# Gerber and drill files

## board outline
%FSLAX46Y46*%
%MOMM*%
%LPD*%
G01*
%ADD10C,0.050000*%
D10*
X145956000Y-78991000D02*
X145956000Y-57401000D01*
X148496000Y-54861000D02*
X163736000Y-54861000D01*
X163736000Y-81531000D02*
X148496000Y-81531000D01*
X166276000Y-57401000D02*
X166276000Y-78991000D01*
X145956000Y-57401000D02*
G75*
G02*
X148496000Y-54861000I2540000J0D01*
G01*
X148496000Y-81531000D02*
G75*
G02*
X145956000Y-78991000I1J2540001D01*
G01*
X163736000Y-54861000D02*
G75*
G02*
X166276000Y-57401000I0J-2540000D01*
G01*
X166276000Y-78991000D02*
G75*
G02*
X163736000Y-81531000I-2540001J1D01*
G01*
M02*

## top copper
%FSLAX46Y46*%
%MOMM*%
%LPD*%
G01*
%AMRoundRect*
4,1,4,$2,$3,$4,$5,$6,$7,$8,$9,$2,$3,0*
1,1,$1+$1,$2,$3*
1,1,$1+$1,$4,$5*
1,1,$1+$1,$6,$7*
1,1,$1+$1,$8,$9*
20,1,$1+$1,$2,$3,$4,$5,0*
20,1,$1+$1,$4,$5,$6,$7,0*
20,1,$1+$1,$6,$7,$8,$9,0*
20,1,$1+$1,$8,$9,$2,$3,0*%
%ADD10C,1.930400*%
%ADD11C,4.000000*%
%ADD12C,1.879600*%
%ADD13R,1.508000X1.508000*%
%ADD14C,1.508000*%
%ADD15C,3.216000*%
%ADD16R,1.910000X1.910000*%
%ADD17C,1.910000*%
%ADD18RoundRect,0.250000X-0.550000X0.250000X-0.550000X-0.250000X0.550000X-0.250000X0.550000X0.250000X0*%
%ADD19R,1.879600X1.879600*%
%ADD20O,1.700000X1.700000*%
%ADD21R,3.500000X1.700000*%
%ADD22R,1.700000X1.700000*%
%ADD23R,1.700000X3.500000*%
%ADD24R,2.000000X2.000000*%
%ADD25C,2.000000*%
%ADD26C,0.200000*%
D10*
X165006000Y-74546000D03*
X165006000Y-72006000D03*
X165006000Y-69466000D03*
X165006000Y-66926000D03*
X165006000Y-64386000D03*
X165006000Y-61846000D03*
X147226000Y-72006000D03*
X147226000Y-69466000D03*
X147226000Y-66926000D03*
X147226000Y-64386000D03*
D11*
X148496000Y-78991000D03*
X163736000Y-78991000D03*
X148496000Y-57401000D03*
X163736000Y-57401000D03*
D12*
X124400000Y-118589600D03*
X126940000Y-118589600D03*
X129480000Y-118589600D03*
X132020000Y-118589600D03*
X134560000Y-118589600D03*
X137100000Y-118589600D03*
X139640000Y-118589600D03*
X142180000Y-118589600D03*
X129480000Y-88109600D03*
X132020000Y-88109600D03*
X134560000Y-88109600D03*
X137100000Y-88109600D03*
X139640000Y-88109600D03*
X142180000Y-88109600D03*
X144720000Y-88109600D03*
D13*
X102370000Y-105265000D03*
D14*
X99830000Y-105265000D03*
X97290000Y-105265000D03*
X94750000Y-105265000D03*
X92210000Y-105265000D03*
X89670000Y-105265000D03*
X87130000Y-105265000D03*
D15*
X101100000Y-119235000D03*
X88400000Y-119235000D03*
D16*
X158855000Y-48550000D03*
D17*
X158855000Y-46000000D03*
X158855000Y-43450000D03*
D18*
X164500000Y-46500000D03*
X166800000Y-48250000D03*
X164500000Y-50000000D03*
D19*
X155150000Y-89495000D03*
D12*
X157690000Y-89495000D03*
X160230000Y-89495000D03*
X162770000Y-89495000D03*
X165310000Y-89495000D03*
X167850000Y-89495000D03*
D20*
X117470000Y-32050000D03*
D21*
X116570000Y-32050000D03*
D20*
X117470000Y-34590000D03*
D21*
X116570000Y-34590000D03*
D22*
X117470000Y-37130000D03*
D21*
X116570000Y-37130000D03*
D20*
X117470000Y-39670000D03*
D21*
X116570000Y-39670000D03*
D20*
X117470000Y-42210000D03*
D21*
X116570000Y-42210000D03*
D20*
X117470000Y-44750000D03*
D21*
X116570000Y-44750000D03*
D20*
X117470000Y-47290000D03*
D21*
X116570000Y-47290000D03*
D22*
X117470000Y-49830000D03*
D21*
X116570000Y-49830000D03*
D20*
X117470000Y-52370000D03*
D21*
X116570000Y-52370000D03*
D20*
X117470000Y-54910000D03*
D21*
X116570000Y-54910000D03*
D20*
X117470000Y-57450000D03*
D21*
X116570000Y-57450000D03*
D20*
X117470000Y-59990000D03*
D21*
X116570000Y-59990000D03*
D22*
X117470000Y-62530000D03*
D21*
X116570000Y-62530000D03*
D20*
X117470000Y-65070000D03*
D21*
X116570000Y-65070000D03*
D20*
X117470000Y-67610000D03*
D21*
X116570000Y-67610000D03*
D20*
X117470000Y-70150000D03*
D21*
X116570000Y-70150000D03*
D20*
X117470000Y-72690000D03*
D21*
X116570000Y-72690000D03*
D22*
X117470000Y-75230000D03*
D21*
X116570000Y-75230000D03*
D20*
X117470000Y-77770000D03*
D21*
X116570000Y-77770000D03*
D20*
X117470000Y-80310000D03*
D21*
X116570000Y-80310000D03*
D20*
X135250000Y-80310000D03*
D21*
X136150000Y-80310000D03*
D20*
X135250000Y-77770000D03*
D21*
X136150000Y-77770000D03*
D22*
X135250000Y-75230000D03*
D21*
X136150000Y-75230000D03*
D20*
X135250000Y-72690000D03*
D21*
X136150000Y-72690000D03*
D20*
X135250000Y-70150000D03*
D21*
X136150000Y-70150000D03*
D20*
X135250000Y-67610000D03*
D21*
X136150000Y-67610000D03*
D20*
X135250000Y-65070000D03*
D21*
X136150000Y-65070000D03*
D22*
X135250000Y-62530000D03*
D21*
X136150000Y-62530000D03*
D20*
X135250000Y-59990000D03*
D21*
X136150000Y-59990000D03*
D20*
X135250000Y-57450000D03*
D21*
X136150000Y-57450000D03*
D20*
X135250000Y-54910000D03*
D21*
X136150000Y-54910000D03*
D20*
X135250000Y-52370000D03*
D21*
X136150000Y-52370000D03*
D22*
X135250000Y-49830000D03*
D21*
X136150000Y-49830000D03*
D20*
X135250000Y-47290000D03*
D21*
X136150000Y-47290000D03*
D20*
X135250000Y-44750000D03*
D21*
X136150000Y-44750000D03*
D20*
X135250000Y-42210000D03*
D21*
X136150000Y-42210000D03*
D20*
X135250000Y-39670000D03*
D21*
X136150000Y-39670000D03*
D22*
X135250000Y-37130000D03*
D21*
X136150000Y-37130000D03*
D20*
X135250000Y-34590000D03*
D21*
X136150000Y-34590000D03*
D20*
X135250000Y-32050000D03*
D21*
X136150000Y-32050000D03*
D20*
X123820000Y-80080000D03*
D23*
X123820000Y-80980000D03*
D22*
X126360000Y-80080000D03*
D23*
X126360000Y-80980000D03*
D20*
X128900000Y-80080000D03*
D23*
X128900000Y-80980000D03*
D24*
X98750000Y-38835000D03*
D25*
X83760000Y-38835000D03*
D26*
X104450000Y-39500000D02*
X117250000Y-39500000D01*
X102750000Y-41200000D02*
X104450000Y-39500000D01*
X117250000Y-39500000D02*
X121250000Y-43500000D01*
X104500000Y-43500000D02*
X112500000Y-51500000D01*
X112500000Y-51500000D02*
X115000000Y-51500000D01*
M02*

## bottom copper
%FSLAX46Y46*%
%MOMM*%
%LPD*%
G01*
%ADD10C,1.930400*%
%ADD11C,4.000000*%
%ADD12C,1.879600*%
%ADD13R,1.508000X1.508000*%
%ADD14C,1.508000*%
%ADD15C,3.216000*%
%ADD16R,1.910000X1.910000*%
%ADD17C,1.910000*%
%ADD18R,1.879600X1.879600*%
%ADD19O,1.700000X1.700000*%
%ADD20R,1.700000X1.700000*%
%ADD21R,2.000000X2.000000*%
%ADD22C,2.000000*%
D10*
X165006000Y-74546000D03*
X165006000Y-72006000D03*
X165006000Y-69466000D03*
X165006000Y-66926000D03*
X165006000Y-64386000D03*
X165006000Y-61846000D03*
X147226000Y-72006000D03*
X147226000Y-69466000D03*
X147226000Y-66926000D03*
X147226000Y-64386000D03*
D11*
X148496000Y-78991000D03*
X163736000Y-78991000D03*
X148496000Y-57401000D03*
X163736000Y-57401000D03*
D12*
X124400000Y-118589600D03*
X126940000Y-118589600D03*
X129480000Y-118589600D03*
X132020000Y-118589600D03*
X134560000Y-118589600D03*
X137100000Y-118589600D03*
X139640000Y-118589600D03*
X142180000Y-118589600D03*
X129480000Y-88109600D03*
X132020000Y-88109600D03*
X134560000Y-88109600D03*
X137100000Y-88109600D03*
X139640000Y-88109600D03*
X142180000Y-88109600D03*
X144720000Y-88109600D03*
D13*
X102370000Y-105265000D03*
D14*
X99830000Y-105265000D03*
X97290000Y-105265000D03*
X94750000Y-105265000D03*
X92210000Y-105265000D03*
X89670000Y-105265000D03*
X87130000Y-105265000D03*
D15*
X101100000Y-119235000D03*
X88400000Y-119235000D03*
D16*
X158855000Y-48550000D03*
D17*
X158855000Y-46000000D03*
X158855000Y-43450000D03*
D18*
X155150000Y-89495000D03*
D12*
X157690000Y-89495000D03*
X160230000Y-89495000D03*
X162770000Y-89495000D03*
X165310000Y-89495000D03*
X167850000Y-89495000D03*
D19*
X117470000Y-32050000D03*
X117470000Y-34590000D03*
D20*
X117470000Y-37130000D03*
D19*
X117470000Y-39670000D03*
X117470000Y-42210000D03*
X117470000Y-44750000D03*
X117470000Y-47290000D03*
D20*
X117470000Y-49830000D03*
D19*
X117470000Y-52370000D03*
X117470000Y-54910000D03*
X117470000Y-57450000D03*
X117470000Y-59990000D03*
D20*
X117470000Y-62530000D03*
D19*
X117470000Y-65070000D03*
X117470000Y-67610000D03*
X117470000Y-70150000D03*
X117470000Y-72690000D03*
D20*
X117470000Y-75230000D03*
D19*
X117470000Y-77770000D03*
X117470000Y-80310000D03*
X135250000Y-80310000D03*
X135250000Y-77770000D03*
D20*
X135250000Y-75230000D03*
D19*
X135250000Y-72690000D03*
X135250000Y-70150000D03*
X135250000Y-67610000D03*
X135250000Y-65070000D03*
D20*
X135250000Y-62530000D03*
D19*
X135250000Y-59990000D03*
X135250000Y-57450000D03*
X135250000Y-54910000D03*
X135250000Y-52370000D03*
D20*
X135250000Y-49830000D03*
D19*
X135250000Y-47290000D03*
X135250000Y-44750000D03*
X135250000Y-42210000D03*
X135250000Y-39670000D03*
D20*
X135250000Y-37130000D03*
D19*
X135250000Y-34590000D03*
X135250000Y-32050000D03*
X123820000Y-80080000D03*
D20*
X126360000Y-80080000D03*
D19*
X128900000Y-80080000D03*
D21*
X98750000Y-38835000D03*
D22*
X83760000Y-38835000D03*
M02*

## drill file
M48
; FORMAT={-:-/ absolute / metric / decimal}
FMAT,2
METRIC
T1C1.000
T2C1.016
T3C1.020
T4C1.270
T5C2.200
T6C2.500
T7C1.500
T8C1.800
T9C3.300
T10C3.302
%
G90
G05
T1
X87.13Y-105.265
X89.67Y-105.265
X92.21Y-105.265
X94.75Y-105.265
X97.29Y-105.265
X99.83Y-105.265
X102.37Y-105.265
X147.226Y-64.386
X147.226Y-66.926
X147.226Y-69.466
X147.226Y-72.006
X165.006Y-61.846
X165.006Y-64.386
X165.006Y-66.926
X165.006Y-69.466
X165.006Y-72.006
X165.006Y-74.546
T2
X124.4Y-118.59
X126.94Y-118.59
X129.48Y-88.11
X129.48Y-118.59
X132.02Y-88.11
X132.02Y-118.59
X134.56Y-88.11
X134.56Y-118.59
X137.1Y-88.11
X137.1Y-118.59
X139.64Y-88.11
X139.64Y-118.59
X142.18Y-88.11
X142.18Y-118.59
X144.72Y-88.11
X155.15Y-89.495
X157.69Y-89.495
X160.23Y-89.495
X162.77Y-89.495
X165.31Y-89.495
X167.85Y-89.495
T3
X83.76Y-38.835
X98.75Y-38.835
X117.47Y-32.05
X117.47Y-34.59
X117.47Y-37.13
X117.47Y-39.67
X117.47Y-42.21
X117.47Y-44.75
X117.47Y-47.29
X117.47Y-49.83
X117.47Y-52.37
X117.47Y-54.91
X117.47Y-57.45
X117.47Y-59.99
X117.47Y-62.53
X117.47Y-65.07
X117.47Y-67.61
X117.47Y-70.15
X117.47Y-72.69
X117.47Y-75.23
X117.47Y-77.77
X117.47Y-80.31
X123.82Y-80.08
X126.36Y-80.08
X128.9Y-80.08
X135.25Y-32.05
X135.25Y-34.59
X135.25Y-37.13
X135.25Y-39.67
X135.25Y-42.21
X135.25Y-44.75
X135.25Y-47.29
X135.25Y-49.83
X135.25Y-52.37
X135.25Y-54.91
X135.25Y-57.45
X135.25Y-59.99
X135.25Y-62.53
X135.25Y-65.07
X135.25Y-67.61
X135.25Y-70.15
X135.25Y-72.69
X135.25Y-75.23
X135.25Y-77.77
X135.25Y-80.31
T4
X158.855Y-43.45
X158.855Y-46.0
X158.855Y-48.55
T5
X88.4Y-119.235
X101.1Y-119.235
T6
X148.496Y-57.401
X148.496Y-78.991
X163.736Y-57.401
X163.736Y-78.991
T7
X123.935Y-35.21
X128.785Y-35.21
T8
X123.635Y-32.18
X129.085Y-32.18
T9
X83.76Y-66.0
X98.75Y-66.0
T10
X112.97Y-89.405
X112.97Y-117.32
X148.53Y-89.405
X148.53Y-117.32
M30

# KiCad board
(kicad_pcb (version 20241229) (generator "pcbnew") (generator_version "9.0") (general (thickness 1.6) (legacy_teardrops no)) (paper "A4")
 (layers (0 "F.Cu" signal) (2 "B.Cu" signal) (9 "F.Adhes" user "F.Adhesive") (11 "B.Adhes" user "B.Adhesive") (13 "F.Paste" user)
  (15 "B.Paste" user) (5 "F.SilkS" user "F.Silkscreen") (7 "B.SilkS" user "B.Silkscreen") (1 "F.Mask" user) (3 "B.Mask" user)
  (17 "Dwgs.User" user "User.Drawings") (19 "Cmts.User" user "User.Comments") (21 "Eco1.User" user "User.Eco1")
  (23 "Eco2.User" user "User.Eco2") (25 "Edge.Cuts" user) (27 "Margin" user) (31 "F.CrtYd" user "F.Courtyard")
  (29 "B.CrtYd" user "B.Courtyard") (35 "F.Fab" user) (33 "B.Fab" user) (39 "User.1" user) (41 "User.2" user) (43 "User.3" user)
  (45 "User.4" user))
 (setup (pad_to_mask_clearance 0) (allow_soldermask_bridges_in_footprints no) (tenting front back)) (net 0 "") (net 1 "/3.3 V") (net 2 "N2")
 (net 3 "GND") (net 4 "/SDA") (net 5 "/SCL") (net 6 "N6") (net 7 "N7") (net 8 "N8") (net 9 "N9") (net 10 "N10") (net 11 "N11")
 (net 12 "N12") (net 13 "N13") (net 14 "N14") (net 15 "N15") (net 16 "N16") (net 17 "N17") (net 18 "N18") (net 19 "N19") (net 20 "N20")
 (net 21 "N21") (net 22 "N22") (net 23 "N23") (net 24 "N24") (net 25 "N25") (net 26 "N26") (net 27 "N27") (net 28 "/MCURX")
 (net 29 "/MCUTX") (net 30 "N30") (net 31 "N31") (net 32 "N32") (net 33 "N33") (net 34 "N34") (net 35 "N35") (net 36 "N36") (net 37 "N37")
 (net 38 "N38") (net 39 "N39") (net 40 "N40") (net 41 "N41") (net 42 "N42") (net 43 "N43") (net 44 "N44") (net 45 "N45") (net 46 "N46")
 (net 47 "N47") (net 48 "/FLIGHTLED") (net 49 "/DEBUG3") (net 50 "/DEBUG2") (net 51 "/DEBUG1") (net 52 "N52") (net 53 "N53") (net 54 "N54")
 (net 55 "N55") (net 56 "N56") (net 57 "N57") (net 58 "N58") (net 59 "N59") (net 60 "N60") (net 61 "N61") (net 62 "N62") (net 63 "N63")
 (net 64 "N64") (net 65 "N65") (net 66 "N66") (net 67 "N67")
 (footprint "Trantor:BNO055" (layer "F.Cu") (at 156.75 67.75 90)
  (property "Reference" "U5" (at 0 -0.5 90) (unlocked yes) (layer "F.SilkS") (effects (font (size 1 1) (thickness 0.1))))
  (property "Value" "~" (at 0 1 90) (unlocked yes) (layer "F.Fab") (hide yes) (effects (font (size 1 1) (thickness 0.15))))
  (fp_line (start -11.241 -10.794) (end 10.349 -10.794) (stroke (width 0.05) (type solid)) (layer "Edge.Cuts"))
  (fp_line (start 12.889 -8.254) (end 12.889 6.986) (stroke (width 0.05) (type solid)) (layer "Edge.Cuts"))
  (fp_line (start -13.781 6.986) (end -13.781 -8.254) (stroke (width 0.05) (type solid)) (layer "Edge.Cuts"))
  (fp_line (start 10.349 9.526) (end -11.241 9.526) (stroke (width 0.05) (type solid)) (layer "Edge.Cuts"))
  (fp_arc (start 10.349 -10.794) (mid 12.145051 -10.050051) (end 12.889 -8.254) (stroke (width 0.05) (type solid)) (layer "Edge.Cuts"))
  (fp_arc (start -13.781 -8.254) (mid -13.037051 -10.050051) (end -11.241 -10.794) (stroke (width 0.05) (type solid)) (layer "Edge.Cuts"))
  (fp_arc (start 12.889 6.986) (mid 12.145051 8.782051) (end 10.349 9.526) (stroke (width 0.05) (type solid)) (layer "Edge.Cuts"))
  (fp_arc (start -11.241 9.526) (mid -13.037051 8.782051) (end -13.781 6.986) (stroke (width 0.05) (type solid)) (layer "Edge.Cuts"))
  (pad "1" thru_hole circle (at -6.796 8.256 180) (size 1.9304 1.9304) (drill 1) (layers "*.Cu" "*.Mask") (remove_unused_layers no)
   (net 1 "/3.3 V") (solder_mask_margin 0.0508) (thermal_bridge_angle 0))
  (pad "2" thru_hole circle (at -4.256 8.256 180) (size 1.9304 1.9304) (drill 1) (layers "*.Cu" "*.Mask") (remove_unused_layers no)
   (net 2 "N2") (solder_mask_margin 0.0508) (thermal_bridge_angle 0))
  (pad "3" thru_hole circle (at -1.716 8.256 180) (size 1.9304 1.9304) (drill 1) (layers "*.Cu" "*.Mask") (remove_unused_layers no)
   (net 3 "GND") (solder_mask_margin 0.0508) (thermal_bridge_angle 0))
  (pad "4" thru_hole circle (at 0.824 8.256 180) (size 1.9304 1.9304) (drill 1) (layers "*.Cu" "*.Mask") (remove_unused_layers no)
   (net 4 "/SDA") (solder_mask_margin 0.0508) (thermal_bridge_angle 0))
  (pad "5" thru_hole circle (at 3.364 8.256 180) (size 1.9304 1.9304) (drill 1) (layers "*.Cu" "*.Mask") (remove_unused_layers no)
   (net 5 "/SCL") (solder_mask_margin 0.0508) (thermal_bridge_angle 0))
  (pad "6" thru_hole circle (at 5.904 8.256 180) (size 1.9304 1.9304) (drill 1) (layers "*.Cu" "*.Mask") (remove_unused_layers no)
   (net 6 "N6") (solder_mask_margin 0.0508) (thermal_bridge_angle 0))
  (pad "7" thru_hole circle (at -4.256 -9.524 180) (size 1.9304 1.9304) (drill 1) (layers "*.Cu" "*.Mask") (remove_unused_layers no)
   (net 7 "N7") (solder_mask_margin 0.0508) (thermal_bridge_angle 0))
  (pad "8" thru_hole circle (at -1.716 -9.524 180) (size 1.9304 1.9304) (drill 1) (layers "*.Cu" "*.Mask") (remove_unused_layers no)
   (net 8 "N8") (solder_mask_margin 0.0508) (thermal_bridge_angle 0))
  (pad "9" thru_hole circle (at 0.824 -9.524 180) (size 1.9304 1.9304) (drill 1) (layers "*.Cu" "*.Mask") (remove_unused_layers no)
   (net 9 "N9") (solder_mask_margin 0.0508) (thermal_bridge_angle 0))
  (pad "10" thru_hole circle (at 3.364 -9.524 180) (size 1.9304 1.9304) (drill 1) (layers "*.Cu" "*.Mask") (remove_unused_layers no)
   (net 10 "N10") (solder_mask_margin 0.0508) (thermal_bridge_angle 0))
  (pad "P$1" thru_hole circle (at -11.241 -8.254 90) (size 4 4) (drill 2.5) (layers "*.Cu" "*.Mask") (remove_unused_layers no)
   (solder_mask_margin 0.0508) (thermal_bridge_angle 0))
  (pad "P$1" thru_hole circle (at -11.241 6.986 90) (size 4 4) (drill 2.5) (layers "*.Cu" "*.Mask") (remove_unused_layers no)
   (solder_mask_margin 0.0508) (thermal_bridge_angle 0))
  (pad "P$1" thru_hole circle (at 10.349 -8.254 90) (size 4 4) (drill 2.5) (layers "*.Cu" "*.Mask") (remove_unused_layers no)
   (solder_mask_margin 0.0508) (thermal_bridge_angle 0))
  (pad "P$1" thru_hole circle (at 10.349 6.986 90) (size 4 4) (drill 2.5) (layers "*.Cu" "*.Mask") (remove_unused_layers no)
   (solder_mask_margin 0.0508) (thermal_bridge_angle 0))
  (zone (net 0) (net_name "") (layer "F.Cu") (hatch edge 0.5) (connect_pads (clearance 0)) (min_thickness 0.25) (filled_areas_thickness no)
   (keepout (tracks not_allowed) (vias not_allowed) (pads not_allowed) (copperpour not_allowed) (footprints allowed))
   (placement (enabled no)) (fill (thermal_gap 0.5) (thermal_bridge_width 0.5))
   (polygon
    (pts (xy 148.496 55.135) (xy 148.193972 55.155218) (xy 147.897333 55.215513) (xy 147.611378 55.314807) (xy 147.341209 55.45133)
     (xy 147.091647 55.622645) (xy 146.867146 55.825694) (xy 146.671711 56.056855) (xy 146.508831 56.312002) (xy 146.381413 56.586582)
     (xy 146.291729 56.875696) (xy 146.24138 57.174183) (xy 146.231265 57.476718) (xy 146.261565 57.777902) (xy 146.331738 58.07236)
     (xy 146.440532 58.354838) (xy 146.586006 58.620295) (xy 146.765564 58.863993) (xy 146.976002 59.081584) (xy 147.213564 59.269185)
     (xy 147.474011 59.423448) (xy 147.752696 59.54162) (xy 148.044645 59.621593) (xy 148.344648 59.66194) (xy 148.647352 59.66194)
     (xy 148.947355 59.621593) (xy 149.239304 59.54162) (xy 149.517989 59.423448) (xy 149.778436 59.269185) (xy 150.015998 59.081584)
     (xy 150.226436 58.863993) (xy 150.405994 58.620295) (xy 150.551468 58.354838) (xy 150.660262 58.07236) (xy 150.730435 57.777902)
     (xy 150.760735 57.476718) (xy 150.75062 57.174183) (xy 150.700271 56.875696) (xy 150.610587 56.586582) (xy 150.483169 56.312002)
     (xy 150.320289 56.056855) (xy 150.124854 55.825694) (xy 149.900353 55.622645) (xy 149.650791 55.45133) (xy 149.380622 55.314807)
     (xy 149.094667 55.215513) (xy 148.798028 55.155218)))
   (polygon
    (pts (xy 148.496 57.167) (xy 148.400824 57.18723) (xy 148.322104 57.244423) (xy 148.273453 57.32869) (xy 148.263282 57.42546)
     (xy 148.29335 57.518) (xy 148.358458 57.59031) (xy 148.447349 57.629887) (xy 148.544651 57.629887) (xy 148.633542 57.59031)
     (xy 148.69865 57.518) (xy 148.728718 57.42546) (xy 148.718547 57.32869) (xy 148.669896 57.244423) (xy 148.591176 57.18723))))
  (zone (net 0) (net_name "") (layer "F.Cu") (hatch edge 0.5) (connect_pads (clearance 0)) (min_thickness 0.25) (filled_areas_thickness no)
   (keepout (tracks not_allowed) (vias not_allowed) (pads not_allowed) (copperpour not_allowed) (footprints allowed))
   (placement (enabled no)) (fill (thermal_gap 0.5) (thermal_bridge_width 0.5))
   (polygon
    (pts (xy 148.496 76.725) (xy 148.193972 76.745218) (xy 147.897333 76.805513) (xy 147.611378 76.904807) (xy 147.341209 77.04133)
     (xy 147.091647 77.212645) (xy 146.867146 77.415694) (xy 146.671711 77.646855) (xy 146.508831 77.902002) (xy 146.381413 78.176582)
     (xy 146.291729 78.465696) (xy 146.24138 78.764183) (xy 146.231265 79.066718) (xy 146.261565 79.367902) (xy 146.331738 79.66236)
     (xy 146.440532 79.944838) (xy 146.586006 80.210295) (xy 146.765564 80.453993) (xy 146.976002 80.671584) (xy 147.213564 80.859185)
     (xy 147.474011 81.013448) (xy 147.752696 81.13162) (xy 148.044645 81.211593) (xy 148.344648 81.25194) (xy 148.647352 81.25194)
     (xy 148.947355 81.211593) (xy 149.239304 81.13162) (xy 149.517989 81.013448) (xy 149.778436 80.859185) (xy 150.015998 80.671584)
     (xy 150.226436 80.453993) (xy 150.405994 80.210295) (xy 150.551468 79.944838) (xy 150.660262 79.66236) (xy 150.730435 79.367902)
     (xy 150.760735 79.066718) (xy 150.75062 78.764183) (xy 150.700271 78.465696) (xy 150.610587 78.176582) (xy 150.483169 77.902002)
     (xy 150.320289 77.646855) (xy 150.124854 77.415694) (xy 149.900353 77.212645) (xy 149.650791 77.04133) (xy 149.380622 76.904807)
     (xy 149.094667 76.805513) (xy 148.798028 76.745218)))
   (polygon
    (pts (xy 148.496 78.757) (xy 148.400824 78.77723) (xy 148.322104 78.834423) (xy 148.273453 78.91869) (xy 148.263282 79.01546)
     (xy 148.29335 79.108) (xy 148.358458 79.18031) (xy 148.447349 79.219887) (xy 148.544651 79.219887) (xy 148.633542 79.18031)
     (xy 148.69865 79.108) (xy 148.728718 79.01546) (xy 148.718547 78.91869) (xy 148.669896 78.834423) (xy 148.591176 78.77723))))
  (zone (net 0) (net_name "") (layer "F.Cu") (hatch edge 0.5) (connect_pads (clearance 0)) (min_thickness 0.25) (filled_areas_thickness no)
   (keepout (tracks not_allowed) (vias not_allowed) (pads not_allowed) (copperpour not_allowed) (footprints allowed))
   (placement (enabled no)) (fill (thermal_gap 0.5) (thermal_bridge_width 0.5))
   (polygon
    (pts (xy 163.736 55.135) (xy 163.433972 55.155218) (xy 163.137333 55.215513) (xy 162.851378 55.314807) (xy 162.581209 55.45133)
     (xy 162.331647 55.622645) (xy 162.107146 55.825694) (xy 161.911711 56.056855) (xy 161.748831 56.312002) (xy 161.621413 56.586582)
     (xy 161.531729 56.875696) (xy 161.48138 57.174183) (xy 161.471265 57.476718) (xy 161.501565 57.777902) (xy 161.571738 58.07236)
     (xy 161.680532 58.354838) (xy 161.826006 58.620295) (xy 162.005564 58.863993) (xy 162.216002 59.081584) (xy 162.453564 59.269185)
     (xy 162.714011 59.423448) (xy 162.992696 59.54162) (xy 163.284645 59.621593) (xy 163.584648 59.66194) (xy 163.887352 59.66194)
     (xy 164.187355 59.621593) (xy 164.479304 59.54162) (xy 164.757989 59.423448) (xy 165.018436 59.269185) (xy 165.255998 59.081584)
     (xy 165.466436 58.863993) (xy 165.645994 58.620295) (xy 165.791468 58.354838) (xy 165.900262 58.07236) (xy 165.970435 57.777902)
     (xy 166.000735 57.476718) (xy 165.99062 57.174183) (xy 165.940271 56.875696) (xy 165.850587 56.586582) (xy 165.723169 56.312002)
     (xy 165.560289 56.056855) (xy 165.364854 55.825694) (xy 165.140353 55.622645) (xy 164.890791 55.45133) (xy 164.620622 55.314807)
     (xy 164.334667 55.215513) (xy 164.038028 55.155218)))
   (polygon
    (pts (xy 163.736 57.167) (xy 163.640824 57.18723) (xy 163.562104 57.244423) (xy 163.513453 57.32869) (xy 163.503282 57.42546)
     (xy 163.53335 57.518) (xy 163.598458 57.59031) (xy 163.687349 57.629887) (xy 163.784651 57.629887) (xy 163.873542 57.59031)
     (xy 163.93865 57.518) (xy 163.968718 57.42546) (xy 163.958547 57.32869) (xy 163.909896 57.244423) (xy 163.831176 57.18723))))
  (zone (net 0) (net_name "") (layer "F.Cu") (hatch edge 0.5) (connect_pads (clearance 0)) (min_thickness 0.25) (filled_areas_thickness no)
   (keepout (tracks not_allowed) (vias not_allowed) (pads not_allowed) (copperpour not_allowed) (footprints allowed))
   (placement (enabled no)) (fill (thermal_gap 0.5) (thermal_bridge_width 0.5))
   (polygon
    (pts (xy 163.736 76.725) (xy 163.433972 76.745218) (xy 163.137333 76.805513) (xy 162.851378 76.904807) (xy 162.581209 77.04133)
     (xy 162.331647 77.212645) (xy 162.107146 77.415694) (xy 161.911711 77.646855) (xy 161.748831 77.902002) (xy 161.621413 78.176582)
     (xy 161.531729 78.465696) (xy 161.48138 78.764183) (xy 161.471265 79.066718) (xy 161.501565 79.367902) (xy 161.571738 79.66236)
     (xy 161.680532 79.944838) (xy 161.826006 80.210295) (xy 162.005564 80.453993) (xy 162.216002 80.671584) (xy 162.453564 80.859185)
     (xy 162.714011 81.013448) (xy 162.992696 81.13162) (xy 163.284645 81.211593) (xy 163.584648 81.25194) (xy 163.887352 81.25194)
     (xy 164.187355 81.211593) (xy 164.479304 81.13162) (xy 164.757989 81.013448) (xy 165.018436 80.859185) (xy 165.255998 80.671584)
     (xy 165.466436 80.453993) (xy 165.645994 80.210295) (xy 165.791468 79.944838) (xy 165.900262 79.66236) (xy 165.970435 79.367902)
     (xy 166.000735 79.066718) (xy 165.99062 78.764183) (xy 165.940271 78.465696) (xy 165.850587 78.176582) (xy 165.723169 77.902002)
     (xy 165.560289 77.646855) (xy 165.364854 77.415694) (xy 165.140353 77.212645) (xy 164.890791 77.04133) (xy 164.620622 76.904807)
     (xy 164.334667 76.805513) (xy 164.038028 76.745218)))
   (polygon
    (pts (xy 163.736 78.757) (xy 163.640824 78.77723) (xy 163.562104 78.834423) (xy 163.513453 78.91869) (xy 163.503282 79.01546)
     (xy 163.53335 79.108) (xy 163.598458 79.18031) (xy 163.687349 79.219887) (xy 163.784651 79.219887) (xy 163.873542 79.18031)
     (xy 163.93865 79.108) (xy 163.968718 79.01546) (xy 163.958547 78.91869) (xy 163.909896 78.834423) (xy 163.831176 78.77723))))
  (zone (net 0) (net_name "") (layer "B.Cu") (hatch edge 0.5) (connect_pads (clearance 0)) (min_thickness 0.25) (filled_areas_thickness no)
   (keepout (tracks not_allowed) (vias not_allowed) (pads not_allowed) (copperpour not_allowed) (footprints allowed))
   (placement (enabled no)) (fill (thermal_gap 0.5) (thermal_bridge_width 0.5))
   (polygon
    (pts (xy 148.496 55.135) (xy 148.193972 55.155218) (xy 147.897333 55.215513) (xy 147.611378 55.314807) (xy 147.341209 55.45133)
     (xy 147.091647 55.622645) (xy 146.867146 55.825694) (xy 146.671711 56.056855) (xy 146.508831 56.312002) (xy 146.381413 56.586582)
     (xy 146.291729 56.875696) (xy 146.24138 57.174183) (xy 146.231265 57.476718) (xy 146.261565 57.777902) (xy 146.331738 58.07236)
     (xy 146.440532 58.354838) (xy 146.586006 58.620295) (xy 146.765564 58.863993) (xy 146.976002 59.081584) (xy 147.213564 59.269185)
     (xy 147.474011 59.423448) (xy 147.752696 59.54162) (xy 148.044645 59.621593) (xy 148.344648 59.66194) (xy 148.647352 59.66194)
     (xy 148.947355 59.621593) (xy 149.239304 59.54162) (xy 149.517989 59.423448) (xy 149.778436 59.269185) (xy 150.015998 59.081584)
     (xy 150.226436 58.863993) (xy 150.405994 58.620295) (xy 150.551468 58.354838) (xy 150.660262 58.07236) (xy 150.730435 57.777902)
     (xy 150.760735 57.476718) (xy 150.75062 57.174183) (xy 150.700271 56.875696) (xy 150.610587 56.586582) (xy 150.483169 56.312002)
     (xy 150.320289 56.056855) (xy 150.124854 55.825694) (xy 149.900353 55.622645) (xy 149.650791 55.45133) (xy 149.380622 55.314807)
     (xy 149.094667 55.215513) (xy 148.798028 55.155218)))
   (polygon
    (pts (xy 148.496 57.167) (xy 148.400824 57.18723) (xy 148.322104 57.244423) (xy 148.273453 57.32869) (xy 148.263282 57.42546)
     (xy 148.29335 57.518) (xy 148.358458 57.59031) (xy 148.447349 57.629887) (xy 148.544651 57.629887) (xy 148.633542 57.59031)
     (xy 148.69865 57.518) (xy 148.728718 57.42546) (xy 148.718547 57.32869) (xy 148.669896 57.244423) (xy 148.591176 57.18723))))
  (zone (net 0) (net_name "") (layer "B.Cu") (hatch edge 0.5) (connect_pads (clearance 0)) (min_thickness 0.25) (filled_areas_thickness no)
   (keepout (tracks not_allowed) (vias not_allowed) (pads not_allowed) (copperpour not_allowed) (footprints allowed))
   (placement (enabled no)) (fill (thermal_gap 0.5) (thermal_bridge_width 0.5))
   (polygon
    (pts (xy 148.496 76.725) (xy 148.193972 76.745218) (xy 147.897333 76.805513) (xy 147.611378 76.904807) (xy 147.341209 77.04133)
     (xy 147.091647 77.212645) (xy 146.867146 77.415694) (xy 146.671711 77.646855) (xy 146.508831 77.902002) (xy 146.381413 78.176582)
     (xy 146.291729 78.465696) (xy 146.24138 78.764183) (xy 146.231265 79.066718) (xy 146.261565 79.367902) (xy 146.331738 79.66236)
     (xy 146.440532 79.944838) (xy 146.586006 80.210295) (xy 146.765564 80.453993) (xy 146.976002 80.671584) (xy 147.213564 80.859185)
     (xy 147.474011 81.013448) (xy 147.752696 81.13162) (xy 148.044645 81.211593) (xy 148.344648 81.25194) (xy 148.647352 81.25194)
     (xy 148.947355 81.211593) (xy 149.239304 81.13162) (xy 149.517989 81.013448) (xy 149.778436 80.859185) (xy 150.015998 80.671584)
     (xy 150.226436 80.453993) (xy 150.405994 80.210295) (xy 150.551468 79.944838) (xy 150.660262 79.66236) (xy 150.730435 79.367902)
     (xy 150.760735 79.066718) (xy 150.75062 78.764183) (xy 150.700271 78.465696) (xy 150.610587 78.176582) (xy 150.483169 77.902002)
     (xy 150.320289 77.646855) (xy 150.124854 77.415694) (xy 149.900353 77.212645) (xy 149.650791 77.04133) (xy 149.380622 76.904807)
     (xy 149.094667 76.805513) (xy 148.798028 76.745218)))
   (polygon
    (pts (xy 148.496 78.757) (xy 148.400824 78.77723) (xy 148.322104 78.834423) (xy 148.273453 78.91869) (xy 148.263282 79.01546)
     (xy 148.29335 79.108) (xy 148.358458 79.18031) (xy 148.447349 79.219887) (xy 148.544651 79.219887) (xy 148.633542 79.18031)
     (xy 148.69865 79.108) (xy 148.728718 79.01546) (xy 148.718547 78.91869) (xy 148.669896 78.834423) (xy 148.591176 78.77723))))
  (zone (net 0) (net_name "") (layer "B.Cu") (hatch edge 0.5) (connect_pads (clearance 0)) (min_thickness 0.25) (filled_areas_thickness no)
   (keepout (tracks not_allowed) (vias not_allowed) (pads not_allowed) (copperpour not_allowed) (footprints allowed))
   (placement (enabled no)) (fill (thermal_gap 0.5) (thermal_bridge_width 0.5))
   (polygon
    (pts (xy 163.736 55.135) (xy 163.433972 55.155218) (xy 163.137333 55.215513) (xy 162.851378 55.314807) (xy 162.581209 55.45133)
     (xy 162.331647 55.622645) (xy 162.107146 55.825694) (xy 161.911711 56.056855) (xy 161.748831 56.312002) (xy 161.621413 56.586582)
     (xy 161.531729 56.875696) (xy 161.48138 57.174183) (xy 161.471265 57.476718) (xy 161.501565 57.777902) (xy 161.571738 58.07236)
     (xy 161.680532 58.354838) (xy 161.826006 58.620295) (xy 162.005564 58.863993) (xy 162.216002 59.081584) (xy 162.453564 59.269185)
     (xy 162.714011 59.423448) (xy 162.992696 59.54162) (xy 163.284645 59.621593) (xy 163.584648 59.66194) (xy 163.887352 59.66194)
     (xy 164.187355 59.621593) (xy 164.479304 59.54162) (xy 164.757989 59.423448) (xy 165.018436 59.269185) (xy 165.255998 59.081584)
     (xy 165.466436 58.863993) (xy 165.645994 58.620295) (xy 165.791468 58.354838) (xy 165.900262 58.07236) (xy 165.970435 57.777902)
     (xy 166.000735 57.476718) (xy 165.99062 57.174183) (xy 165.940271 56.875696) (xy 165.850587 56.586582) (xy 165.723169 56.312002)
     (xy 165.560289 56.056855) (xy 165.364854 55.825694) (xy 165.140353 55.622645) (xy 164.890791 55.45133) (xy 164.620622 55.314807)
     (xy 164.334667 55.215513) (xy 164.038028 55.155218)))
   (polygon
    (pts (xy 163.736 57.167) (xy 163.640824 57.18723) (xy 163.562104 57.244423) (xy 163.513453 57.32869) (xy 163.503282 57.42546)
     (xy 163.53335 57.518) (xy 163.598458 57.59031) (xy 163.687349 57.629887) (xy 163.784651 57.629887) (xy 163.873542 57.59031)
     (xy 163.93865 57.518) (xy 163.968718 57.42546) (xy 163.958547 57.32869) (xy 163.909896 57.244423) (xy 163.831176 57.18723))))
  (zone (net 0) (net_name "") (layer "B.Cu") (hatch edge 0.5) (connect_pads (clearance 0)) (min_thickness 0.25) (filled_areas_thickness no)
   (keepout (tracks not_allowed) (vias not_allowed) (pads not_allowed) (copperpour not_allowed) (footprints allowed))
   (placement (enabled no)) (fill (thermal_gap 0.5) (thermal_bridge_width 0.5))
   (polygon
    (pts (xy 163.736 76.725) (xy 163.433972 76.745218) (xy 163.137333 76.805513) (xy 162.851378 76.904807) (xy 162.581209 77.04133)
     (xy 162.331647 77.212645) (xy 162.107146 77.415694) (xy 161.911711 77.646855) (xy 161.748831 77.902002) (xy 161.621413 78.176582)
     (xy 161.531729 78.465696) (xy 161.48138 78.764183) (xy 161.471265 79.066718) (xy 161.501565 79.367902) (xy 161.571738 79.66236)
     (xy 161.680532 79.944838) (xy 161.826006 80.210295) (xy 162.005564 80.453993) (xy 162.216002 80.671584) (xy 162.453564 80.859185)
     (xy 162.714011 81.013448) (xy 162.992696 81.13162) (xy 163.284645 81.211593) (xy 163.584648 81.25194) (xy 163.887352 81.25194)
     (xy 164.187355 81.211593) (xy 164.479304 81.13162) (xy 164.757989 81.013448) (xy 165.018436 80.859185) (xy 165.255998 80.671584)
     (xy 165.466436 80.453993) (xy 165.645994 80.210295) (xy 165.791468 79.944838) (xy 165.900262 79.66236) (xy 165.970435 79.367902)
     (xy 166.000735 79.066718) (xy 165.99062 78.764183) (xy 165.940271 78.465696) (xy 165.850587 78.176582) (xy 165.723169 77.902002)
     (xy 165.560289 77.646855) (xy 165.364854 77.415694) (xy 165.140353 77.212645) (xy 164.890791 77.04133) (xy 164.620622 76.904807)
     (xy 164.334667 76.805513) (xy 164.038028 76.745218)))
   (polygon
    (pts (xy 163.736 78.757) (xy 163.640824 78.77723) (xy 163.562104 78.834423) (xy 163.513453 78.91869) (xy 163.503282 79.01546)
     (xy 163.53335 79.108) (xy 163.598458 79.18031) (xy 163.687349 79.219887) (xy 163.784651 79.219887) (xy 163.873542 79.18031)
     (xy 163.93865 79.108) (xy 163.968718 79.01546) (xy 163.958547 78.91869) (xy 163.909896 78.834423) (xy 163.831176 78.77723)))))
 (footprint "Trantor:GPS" (layer "F.Cu") (at 141.197 119.9866)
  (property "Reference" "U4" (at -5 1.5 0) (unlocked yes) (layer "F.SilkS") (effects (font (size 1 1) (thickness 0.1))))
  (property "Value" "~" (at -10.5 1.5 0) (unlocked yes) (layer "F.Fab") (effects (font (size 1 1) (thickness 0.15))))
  (pad "" np_thru_hole circle (at -28.227 -30.5816) (size 3.302 3.302) (drill 3.302) (layers "*.Cu" "*.Mask"))
  (pad "" np_thru_hole circle (at -28.227 -2.667) (size 3.302 3.302) (drill 3.302) (layers "*.Cu" "*.Mask"))
  (pad "" np_thru_hole circle (at 7.333 -30.5816) (size 3.302 3.302) (drill 3.302) (layers "*.Cu" "*.Mask"))
  (pad "" np_thru_hole circle (at 7.333 -2.667) (size 3.302 3.302) (drill 3.302) (layers "*.Cu" "*.Mask"))
  (pad "1" thru_hole circle (at -16.797 -1.397 270) (size 1.8796 1.8796) (drill 1.016) (layers "*.Cu" "*.Mask") (remove_unused_layers no)
   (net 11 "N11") (solder_mask_margin 0.1016) (thermal_bridge_angle 0))
  (pad "2" thru_hole circle (at -14.257 -1.397 270) (size 1.8796 1.8796) (drill 1.016) (layers "*.Cu" "*.Mask") (remove_unused_layers no)
   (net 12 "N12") (solder_mask_margin 0.1016) (thermal_bridge_angle 0))
  (pad "3" thru_hole circle (at -11.717 -1.397 270) (size 1.8796 1.8796) (drill 1.016) (layers "*.Cu" "*.Mask") (remove_unused_layers no)
   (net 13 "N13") (solder_mask_margin 0.1016) (thermal_bridge_angle 0))
  (pad "4" thru_hole circle (at -9.177 -1.397 270) (size 1.8796 1.8796) (drill 1.016) (layers "*.Cu" "*.Mask") (remove_unused_layers no)
   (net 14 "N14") (solder_mask_margin 0.1016) (thermal_bridge_angle 0))
  (pad "5" thru_hole circle (at -6.637 -1.397 90) (size 1.8796 1.8796) (drill 1.016) (layers "*.Cu" "*.Mask") (remove_unused_layers no)
   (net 3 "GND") (solder_mask_margin 0.1016) (thermal_bridge_angle 0))
  (pad "6" thru_hole circle (at -4.097 -1.397 90) (size 1.8796 1.8796) (drill 1.016) (layers "*.Cu" "*.Mask") (remove_unused_layers no)
   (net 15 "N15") (solder_mask_margin 0.1016) (thermal_bridge_angle 0))
  (pad "7" thru_hole circle (at -1.557 -1.397 90) (size 1.8796 1.8796) (drill 1.016) (layers "*.Cu" "*.Mask") (remove_unused_layers no)
   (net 4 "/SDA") (solder_mask_margin 0.1016) (thermal_bridge_angle 0))
  (pad "8" thru_hole circle (at 0.983 -1.397 90) (size 1.8796 1.8796) (drill 1.016) (layers "*.Cu" "*.Mask") (remove_unused_layers no)
   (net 5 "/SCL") (solder_mask_margin 0.1016) (thermal_bridge_angle 0))
  (pad "9" thru_hole circle (at -11.717 -31.877 90) (size 1.8796 1.8796) (drill 1.016) (layers "*.Cu" "*.Mask") (remove_unused_layers no)
   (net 3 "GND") (solder_mask_margin 0.1016) (thermal_bridge_angle 0))
  (pad "10" thru_hole circle (at -9.177 -31.877 90) (size 1.8796 1.8796) (drill 1.016) (layers "*.Cu" "*.Mask") (remove_unused_layers no)
   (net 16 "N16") (solder_mask_margin 0.1016) (thermal_bridge_angle 0))
  (pad "11" thru_hole circle (at -6.637 -31.877 90) (size 1.8796 1.8796) (drill 1.016) (layers "*.Cu" "*.Mask") (remove_unused_layers no)
   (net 1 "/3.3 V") (solder_mask_margin 0.1016) (thermal_bridge_angle 0))
  (pad "12" thru_hole circle (at -4.097 -31.877 90) (size 1.8796 1.8796) (drill 1.016) (layers "*.Cu" "*.Mask") (remove_unused_layers no)
   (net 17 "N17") (solder_mask_margin 0.1016) (thermal_bridge_angle 0))
  (pad "13" thru_hole circle (at -1.557 -31.877 90) (size 1.8796 1.8796) (drill 1.016) (layers "*.Cu" "*.Mask") (remove_unused_layers no)
   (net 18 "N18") (solder_mask_margin 0.1016) (thermal_bridge_angle 0))
  (pad "14" thru_hole circle (at 0.983 -31.877 90) (size 1.8796 1.8796) (drill 1.016) (layers "*.Cu" "*.Mask") (remove_unused_layers no)
   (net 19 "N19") (solder_mask_margin 0.1016) (thermal_bridge_angle 0))
  (pad "15" thru_hole circle (at 3.523 -31.877 90) (size 1.8796 1.8796) (drill 1.016) (layers "*.Cu" "*.Mask") (remove_unused_layers no)
   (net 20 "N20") (solder_mask_margin 0.1016) (thermal_bridge_angle 0)))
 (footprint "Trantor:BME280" (layer "F.Cu") (at 94.75 112.25 180)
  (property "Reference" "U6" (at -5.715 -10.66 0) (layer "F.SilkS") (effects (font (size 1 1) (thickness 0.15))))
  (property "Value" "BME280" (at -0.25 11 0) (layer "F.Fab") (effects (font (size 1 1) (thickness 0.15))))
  (pad "1" thru_hole rect (at -7.62 6.985 180) (size 1.508 1.508) (drill 1) (layers "*.Cu" "*.Mask") (remove_unused_layers no)
   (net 1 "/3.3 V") (solder_mask_margin 0.102))
  (pad "2" thru_hole circle (at -5.08 6.985 180) (size 1.508 1.508) (drill 1) (layers "*.Cu" "*.Mask") (remove_unused_layers no)
   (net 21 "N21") (solder_mask_margin 0.102))
  (pad "3" thru_hole circle (at -2.54 6.985 180) (size 1.508 1.508) (drill 1) (layers "*.Cu" "*.Mask") (remove_unused_layers no)
   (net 3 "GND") (solder_mask_margin 0.102))
  (pad "4" thru_hole circle (at 0 6.985 180) (size 1.508 1.508) (drill 1) (layers "*.Cu" "*.Mask") (remove_unused_layers no) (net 5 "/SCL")
   (solder_mask_margin 0.102))
  (pad "5" thru_hole circle (at 2.54 6.985 180) (size 1.508 1.508) (drill 1) (layers "*.Cu" "*.Mask") (remove_unused_layers no)
   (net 4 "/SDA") (solder_mask_margin 0.102))
  (pad "6" thru_hole circle (at 5.08 6.985 180) (size 1.508 1.508) (drill 1) (layers "*.Cu" "*.Mask") (remove_unused_layers no)
   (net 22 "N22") (solder_mask_margin 0.102))
  (pad "7" thru_hole circle (at 7.62 6.985 180) (size 1.508 1.508) (drill 1) (layers "*.Cu" "*.Mask") (remove_unused_layers no)
   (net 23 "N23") (solder_mask_margin 0.102))
  (pad "P1" thru_hole circle (at -6.35 -6.985 180) (size 3.216 3.216) (drill 2.2) (layers "*.Cu" "*.Mask") (remove_unused_layers no)
   (solder_mask_margin 0.102))
  (pad "P2" thru_hole circle (at 6.35 -6.985 180) (size 3.216 3.216) (drill 2.2) (layers "*.Cu" "*.Mask") (remove_unused_layers no)
   (solder_mask_margin 0.102)))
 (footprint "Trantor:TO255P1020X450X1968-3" (layer "F.Cu") (at 158.25 46 90)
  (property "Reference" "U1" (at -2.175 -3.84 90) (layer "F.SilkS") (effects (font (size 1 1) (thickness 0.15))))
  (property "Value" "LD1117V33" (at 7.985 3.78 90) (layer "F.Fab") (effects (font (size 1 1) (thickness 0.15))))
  (pad "1" thru_hole rect (at -2.55 0.605 90) (size 1.91 1.91) (drill 1.27) (layers "*.Cu" "*.Mask") (remove_unused_layers no) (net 3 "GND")
   (solder_mask_margin 0.102))
  (pad "2" thru_hole circle (at 0 0.605 90) (size 1.91 1.91) (drill 1.27) (layers "*.Cu" "*.Mask") (remove_unused_layers no)
   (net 1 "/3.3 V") (solder_mask_margin 0.102))
  (pad "3" thru_hole circle (at 2.55 0.605 90) (size 1.91 1.91) (drill 1.27) (layers "*.Cu" "*.Mask") (remove_unused_layers no)
   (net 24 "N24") (solder_mask_margin 0.102)))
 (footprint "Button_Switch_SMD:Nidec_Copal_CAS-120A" (layer "F.Cu") (at 165.65 48.25)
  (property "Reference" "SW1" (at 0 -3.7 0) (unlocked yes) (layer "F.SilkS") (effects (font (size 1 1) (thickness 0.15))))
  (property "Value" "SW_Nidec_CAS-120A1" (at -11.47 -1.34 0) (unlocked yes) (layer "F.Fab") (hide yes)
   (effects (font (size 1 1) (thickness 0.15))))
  (pad "1" smd roundrect (at -1.15 -1.75 270) (size 1 1.6) (layers "F.Cu" "F.Mask" "F.Paste") (roundrect_rratio 0.25) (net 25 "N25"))
  (pad "2" smd roundrect (at 1.15 0 270) (size 1 1.6) (layers "F.Cu" "F.Mask" "F.Paste") (roundrect_rratio 0.25) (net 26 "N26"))
  (pad "3" smd roundrect (at -1.15 1.75 270) (size 1 1.6) (layers "F.Cu" "F.Mask" "F.Paste") (roundrect_rratio 0.25) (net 24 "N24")))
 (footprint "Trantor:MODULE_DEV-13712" (layer "F.Cu") (at 161.5 97.75 180)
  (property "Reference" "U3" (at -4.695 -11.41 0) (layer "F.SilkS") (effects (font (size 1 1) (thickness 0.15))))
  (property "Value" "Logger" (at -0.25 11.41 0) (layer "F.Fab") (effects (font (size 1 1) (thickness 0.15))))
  (pad "1" thru_hole rect (at 6.35 8.255 180) (size 1.8796 1.8796) (drill 1.016) (layers "*.Cu" "*.Mask") (remove_unused_layers no)
   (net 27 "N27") (solder_mask_margin 0.102))
  (pad "2" thru_hole circle (at 3.81 8.255 180) (size 1.8796 1.8796) (drill 1.016) (layers "*.Cu" "*.Mask") (remove_unused_layers no)
   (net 3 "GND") (solder_mask_margin 0.102))
  (pad "3" thru_hole circle (at 1.27 8.255 180) (size 1.8796 1.8796) (drill 1.016) (layers "*.Cu" "*.Mask") (remove_unused_layers no)
   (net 1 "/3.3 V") (solder_mask_margin 0.102))
  (pad "4" thru_hole circle (at -1.27 8.255 180) (size 1.8796 1.8796) (drill 1.016) (layers "*.Cu" "*.Mask") (remove_unused_layers no)
   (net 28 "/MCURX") (solder_mask_margin 0.102))
  (pad "5" thru_hole circle (at -3.81 8.255 180) (size 1.8796 1.8796) (drill 1.016) (layers "*.Cu" "*.Mask") (remove_unused_layers no)
   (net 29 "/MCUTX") (solder_mask_margin 0.102))
  (pad "6" thru_hole circle (at -6.35 8.255 180) (size 1.8796 1.8796) (drill 1.016) (layers "*.Cu" "*.Mask") (remove_unused_layers no)
   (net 3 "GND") (solder_mask_margin 0.102)))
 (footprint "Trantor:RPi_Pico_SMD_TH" (layer "F.Cu") (at 126.36 56.18)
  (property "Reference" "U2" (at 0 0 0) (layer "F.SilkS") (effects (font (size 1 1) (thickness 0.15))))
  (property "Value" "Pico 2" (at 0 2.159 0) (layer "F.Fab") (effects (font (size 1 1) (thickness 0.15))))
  (pad "" np_thru_hole oval (at -2.725 -24) (size 1.8 1.8) (drill 1.8) (layers "*.Cu" "*.Mask"))
  (pad "" np_thru_hole oval (at -2.425 -20.97) (size 1.5 1.5) (drill 1.5) (layers "*.Cu" "*.Mask"))
  (pad "" np_thru_hole oval (at 2.425 -20.97) (size 1.5 1.5) (drill 1.5) (layers "*.Cu" "*.Mask"))
  (pad "" np_thru_hole oval (at 2.725 -24) (size 1.8 1.8) (drill 1.8) (layers "*.Cu" "*.Mask"))
  (pad "1" thru_hole oval (at -8.89 -24.13) (size 1.7 1.7) (drill 1.02) (layers "*.Cu" "*.Mask") (remove_unused_layers no) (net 29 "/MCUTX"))
  (pad "1" smd rect (at -8.89 -24.13) (size 3.5 1.7) (drill (offset -0.9 0)) (layers "F.Cu" "F.Mask") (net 29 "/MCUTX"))
  (pad "2" thru_hole oval (at -8.89 -21.59) (size 1.7 1.7) (drill 1.02) (layers "*.Cu" "*.Mask") (remove_unused_layers no) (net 28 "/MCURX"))
  (pad "2" smd rect (at -8.89 -21.59) (size 3.5 1.7) (drill (offset -0.9 0)) (layers "F.Cu" "F.Mask") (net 28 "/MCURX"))
  (pad "3" thru_hole rect (at -8.89 -19.05) (size 1.7 1.7) (drill 1.02) (layers "*.Cu" "*.Mask") (remove_unused_layers no) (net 3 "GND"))
  (pad "3" smd rect (at -8.89 -19.05) (size 3.5 1.7) (drill (offset -0.9 0)) (layers "F.Cu" "F.Mask") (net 3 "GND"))
  (pad "4" thru_hole oval (at -8.89 -16.51) (size 1.7 1.7) (drill 1.02) (layers "*.Cu" "*.Mask") (remove_unused_layers no) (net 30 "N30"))
  (pad "4" smd rect (at -8.89 -16.51) (size 3.5 1.7) (drill (offset -0.9 0)) (layers "F.Cu" "F.Mask") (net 30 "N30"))
  (pad "5" thru_hole oval (at -8.89 -13.97) (size 1.7 1.7) (drill 1.02) (layers "*.Cu" "*.Mask") (remove_unused_layers no) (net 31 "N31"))
  (pad "5" smd rect (at -8.89 -13.97) (size 3.5 1.7) (drill (offset -0.9 0)) (layers "F.Cu" "F.Mask") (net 31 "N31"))
  (pad "6" thru_hole oval (at -8.89 -11.43) (size 1.7 1.7) (drill 1.02) (layers "*.Cu" "*.Mask") (remove_unused_layers no) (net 4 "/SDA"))
  (pad "6" smd rect (at -8.89 -11.43) (size 3.5 1.7) (drill (offset -0.9 0)) (layers "F.Cu" "F.Mask") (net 4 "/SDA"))
  (pad "7" thru_hole oval (at -8.89 -8.89) (size 1.7 1.7) (drill 1.02) (layers "*.Cu" "*.Mask") (remove_unused_layers no) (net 5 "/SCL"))
  (pad "7" smd rect (at -8.89 -8.89) (size 3.5 1.7) (drill (offset -0.9 0)) (layers "F.Cu" "F.Mask") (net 5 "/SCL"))
  (pad "8" thru_hole rect (at -8.89 -6.35) (size 1.7 1.7) (drill 1.02) (layers "*.Cu" "*.Mask") (remove_unused_layers no) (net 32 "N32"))
  (pad "8" smd rect (at -8.89 -6.35) (size 3.5 1.7) (drill (offset -0.9 0)) (layers "F.Cu" "F.Mask") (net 32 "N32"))
  (pad "9" thru_hole oval (at -8.89 -3.81) (size 1.7 1.7) (drill 1.02) (layers "*.Cu" "*.Mask") (remove_unused_layers no) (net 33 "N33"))
  (pad "9" smd rect (at -8.89 -3.81) (size 3.5 1.7) (drill (offset -0.9 0)) (layers "F.Cu" "F.Mask") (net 33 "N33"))
  (pad "10" thru_hole oval (at -8.89 -1.27) (size 1.7 1.7) (drill 1.02) (layers "*.Cu" "*.Mask") (remove_unused_layers no) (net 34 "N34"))
  (pad "10" smd rect (at -8.89 -1.27) (size 3.5 1.7) (drill (offset -0.9 0)) (layers "F.Cu" "F.Mask") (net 34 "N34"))
  (pad "11" thru_hole oval (at -8.89 1.27) (size 1.7 1.7) (drill 1.02) (layers "*.Cu" "*.Mask") (remove_unused_layers no) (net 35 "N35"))
  (pad "11" smd rect (at -8.89 1.27) (size 3.5 1.7) (drill (offset -0.9 0)) (layers "F.Cu" "F.Mask") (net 35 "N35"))
  (pad "12" thru_hole oval (at -8.89 3.81) (size 1.7 1.7) (drill 1.02) (layers "*.Cu" "*.Mask") (remove_unused_layers no) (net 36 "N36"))
  (pad "12" smd rect (at -8.89 3.81) (size 3.5 1.7) (drill (offset -0.9 0)) (layers "F.Cu" "F.Mask") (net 36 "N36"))
  (pad "13" thru_hole rect (at -8.89 6.35) (size 1.7 1.7) (drill 1.02) (layers "*.Cu" "*.Mask") (remove_unused_layers no) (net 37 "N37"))
  (pad "13" smd rect (at -8.89 6.35) (size 3.5 1.7) (drill (offset -0.9 0)) (layers "F.Cu" "F.Mask") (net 37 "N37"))
  (pad "14" thru_hole oval (at -8.89 8.89) (size 1.7 1.7) (drill 1.02) (layers "*.Cu" "*.Mask") (remove_unused_layers no) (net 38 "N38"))
  (pad "14" smd rect (at -8.89 8.89) (size 3.5 1.7) (drill (offset -0.9 0)) (layers "F.Cu" "F.Mask") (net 38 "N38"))
  (pad "15" thru_hole oval (at -8.89 11.43) (size 1.7 1.7) (drill 1.02) (layers "*.Cu" "*.Mask") (remove_unused_layers no) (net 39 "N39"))
  (pad "15" smd rect (at -8.89 11.43) (size 3.5 1.7) (drill (offset -0.9 0)) (layers "F.Cu" "F.Mask") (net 39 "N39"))
  (pad "16" thru_hole oval (at -8.89 13.97) (size 1.7 1.7) (drill 1.02) (layers "*.Cu" "*.Mask") (remove_unused_layers no) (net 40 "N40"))
  (pad "16" smd rect (at -8.89 13.97) (size 3.5 1.7) (drill (offset -0.9 0)) (layers "F.Cu" "F.Mask") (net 40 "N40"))
  (pad "17" thru_hole oval (at -8.89 16.51) (size 1.7 1.7) (drill 1.02) (layers "*.Cu" "*.Mask") (remove_unused_layers no) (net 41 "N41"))
  (pad "17" smd rect (at -8.89 16.51) (size 3.5 1.7) (drill (offset -0.9 0)) (layers "F.Cu" "F.Mask") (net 41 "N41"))
  (pad "18" thru_hole rect (at -8.89 19.05) (size 1.7 1.7) (drill 1.02) (layers "*.Cu" "*.Mask") (remove_unused_layers no) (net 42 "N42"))
  (pad "18" smd rect (at -8.89 19.05) (size 3.5 1.7) (drill (offset -0.9 0)) (layers "F.Cu" "F.Mask") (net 42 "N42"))
  (pad "19" thru_hole oval (at -8.89 21.59) (size 1.7 1.7) (drill 1.02) (layers "*.Cu" "*.Mask") (remove_unused_layers no) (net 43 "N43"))
  (pad "19" smd rect (at -8.89 21.59) (size 3.5 1.7) (drill (offset -0.9 0)) (layers "F.Cu" "F.Mask") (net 43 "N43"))
  (pad "20" thru_hole oval (at -8.89 24.13) (size 1.7 1.7) (drill 1.02) (layers "*.Cu" "*.Mask") (remove_unused_layers no) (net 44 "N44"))
  (pad "20" smd rect (at -8.89 24.13) (size 3.5 1.7) (drill (offset -0.9 0)) (layers "F.Cu" "F.Mask") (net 44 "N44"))
  (pad "21" thru_hole oval (at 8.89 24.13) (size 1.7 1.7) (drill 1.02) (layers "*.Cu" "*.Mask") (remove_unused_layers no) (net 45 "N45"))
  (pad "21" smd rect (at 8.89 24.13) (size 3.5 1.7) (drill (offset 0.9 0)) (layers "F.Cu" "F.Mask") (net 45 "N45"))
  (pad "22" thru_hole oval (at 8.89 21.59) (size 1.7 1.7) (drill 1.02) (layers "*.Cu" "*.Mask") (remove_unused_layers no) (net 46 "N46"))
  (pad "22" smd rect (at 8.89 21.59) (size 3.5 1.7) (drill (offset 0.9 0)) (layers "F.Cu" "F.Mask") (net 46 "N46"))
  (pad "23" thru_hole rect (at 8.89 19.05) (size 1.7 1.7) (drill 1.02) (layers "*.Cu" "*.Mask") (remove_unused_layers no) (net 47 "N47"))
  (pad "23" smd rect (at 8.89 19.05) (size 3.5 1.7) (drill (offset 0.9 0)) (layers "F.Cu" "F.Mask") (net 47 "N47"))
  (pad "24" thru_hole oval (at 8.89 16.51) (size 1.7 1.7) (drill 1.02) (layers "*.Cu" "*.Mask") (remove_unused_layers no)
   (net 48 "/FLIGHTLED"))
  (pad "24" smd rect (at 8.89 16.51) (size 3.5 1.7) (drill (offset 0.9 0)) (layers "F.Cu" "F.Mask") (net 48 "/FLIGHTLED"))
  (pad "25" thru_hole oval (at 8.89 13.97) (size 1.7 1.7) (drill 1.02) (layers "*.Cu" "*.Mask") (remove_unused_layers no) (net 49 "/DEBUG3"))
  (pad "25" smd rect (at 8.89 13.97) (size 3.5 1.7) (drill (offset 0.9 0)) (layers "F.Cu" "F.Mask") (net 49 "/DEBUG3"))
  (pad "26" thru_hole oval (at 8.89 11.43) (size 1.7 1.7) (drill 1.02) (layers "*.Cu" "*.Mask") (remove_unused_layers no) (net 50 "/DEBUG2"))
  (pad "26" smd rect (at 8.89 11.43) (size 3.5 1.7) (drill (offset 0.9 0)) (layers "F.Cu" "F.Mask") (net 50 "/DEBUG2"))
  (pad "27" thru_hole oval (at 8.89 8.89) (size 1.7 1.7) (drill 1.02) (layers "*.Cu" "*.Mask") (remove_unused_layers no) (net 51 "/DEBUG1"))
  (pad "27" smd rect (at 8.89 8.89) (size 3.5 1.7) (drill (offset 0.9 0)) (layers "F.Cu" "F.Mask") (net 51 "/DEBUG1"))
  (pad "28" thru_hole rect (at 8.89 6.35) (size 1.7 1.7) (drill 1.02) (layers "*.Cu" "*.Mask") (remove_unused_layers no) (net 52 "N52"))
  (pad "28" smd rect (at 8.89 6.35) (size 3.5 1.7) (drill (offset 0.9 0)) (layers "F.Cu" "F.Mask") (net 52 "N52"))
  (pad "29" thru_hole oval (at 8.89 3.81) (size 1.7 1.7) (drill 1.02) (layers "*.Cu" "*.Mask") (remove_unused_layers no) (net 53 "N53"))
  (pad "29" smd rect (at 8.89 3.81) (size 3.5 1.7) (drill (offset 0.9 0)) (layers "F.Cu" "F.Mask") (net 53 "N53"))
  (pad "30" thru_hole oval (at 8.89 1.27) (size 1.7 1.7) (drill 1.02) (layers "*.Cu" "*.Mask") (remove_unused_layers no) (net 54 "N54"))
  (pad "30" smd rect (at 8.89 1.27) (size 3.5 1.7) (drill (offset 0.9 0)) (layers "F.Cu" "F.Mask") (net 54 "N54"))
  (pad "31" thru_hole oval (at 8.89 -1.27) (size 1.7 1.7) (drill 1.02) (layers "*.Cu" "*.Mask") (remove_unused_layers no) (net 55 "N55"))
  (pad "31" smd rect (at 8.89 -1.27) (size 3.5 1.7) (drill (offset 0.9 0)) (layers "F.Cu" "F.Mask") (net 55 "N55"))
  (pad "32" thru_hole oval (at 8.89 -3.81) (size 1.7 1.7) (drill 1.02) (layers "*.Cu" "*.Mask") (remove_unused_layers no) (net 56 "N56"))
  (pad "32" smd rect (at 8.89 -3.81) (size 3.5 1.7) (drill (offset 0.9 0)) (layers "F.Cu" "F.Mask") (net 56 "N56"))
  (pad "33" thru_hole rect (at 8.89 -6.35) (size 1.7 1.7) (drill 1.02) (layers "*.Cu" "*.Mask") (remove_unused_layers no) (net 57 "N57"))
  (pad "33" smd rect (at 8.89 -6.35) (size 3.5 1.7) (drill (offset 0.9 0)) (layers "F.Cu" "F.Mask") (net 57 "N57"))
  (pad "34" thru_hole oval (at 8.89 -8.89) (size 1.7 1.7) (drill 1.02) (layers "*.Cu" "*.Mask") (remove_unused_layers no) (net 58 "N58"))
  (pad "34" smd rect (at 8.89 -8.89) (size 3.5 1.7) (drill (offset 0.9 0)) (layers "F.Cu" "F.Mask") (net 58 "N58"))
  (pad "35" thru_hole oval (at 8.89 -11.43) (size 1.7 1.7) (drill 1.02) (layers "*.Cu" "*.Mask") (remove_unused_layers no) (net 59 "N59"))
  (pad "35" smd rect (at 8.89 -11.43) (size 3.5 1.7) (drill (offset 0.9 0)) (layers "F.Cu" "F.Mask") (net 59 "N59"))
  (pad "36" thru_hole oval (at 8.89 -13.97) (size 1.7 1.7) (drill 1.02) (layers "*.Cu" "*.Mask") (remove_unused_layers no) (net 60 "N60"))
  (pad "36" smd rect (at 8.89 -13.97) (size 3.5 1.7) (drill (offset 0.9 0)) (layers "F.Cu" "F.Mask") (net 60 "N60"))
  (pad "37" thru_hole oval (at 8.89 -16.51) (size 1.7 1.7) (drill 1.02) (layers "*.Cu" "*.Mask") (remove_unused_layers no) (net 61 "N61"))
  (pad "37" smd rect (at 8.89 -16.51) (size 3.5 1.7) (drill (offset 0.9 0)) (layers "F.Cu" "F.Mask") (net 61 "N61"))
  (pad "38" thru_hole rect (at 8.89 -19.05) (size 1.7 1.7) (drill 1.02) (layers "*.Cu" "*.Mask") (remove_unused_layers no) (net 3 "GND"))
  (pad "38" smd rect (at 8.89 -19.05) (size 3.5 1.7) (drill (offset 0.9 0)) (layers "F.Cu" "F.Mask") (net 3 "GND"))
  (pad "39" thru_hole oval (at 8.89 -21.59) (size 1.7 1.7) (drill 1.02) (layers "*.Cu" "*.Mask") (remove_unused_layers no) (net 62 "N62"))
  (pad "39" smd rect (at 8.89 -21.59) (size 3.5 1.7) (drill (offset 0.9 0)) (layers "F.Cu" "F.Mask") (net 62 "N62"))
  (pad "40" thru_hole oval (at 8.89 -24.13) (size 1.7 1.7) (drill 1.02) (layers "*.Cu" "*.Mask") (remove_unused_layers no) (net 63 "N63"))
  (pad "40" smd rect (at 8.89 -24.13) (size 3.5 1.7) (drill (offset 0.9 0)) (layers "F.Cu" "F.Mask") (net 63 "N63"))
  (pad "41" thru_hole oval (at -2.54 23.9) (size 1.7 1.7) (drill 1.02) (layers "*.Cu" "*.Mask") (remove_unused_layers no) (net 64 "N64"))
  (pad "41" smd rect (at -2.54 23.9 90) (size 3.5 1.7) (drill (offset -0.9 0)) (layers "F.Cu" "F.Mask") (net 64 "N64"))
  (pad "42" thru_hole rect (at 0 23.9) (size 1.7 1.7) (drill 1.02) (layers "*.Cu" "*.Mask") (remove_unused_layers no) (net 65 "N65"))
  (pad "42" smd rect (at 0 23.9 90) (size 3.5 1.7) (drill (offset -0.9 0)) (layers "F.Cu" "F.Mask") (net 65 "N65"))
  (pad "43" thru_hole oval (at 2.54 23.9) (size 1.7 1.7) (drill 1.02) (layers "*.Cu" "*.Mask") (remove_unused_layers no) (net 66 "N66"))
  (pad "43" smd rect (at 2.54 23.9 90) (size 3.5 1.7) (drill (offset -0.9 0)) (layers "F.Cu" "F.Mask") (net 66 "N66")))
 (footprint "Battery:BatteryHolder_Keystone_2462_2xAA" (layer "F.Cu") (at 98.75 38.835 -90)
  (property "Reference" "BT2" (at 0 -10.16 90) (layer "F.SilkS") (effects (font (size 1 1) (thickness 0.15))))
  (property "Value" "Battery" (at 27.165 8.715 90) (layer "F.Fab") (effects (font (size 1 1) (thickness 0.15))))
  (pad "" np_thru_hole circle (at 27.165 0 270) (size 3.3 3.3) (drill 3.3) (layers "*.Cu" "*.Mask"))
  (pad "" np_thru_hole circle (at 27.165 14.99 270) (size 3.3 3.3) (drill 3.3) (layers "*.Cu" "*.Mask"))
  (pad "1" thru_hole rect (at 0 0 270) (size 2 2) (drill 1.02) (layers "*.Cu" "*.Mask") (remove_unused_layers no) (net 26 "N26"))
  (pad "2" thru_hole circle (at 0 14.99 270) (size 2 2) (drill 1.02) (layers "*.Cu" "*.Mask") (remove_unused_layers no) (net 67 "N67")))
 (segment (start 104.45 39.5) (end 117.25 39.5) (width 0.2) (layer "F.Cu") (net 30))
 (segment (start 102.75 41.2) (end 104.45 39.5) (width 0.2) (layer "F.Cu") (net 30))
 (segment (start 117.25 39.5) (end 121.25 43.5) (width 0.2) (layer "F.Cu") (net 30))
 (segment (start 104.5 43.5) (end 112.5 51.5) (width 0.2) (layer "F.Cu") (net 33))
 (segment (start 112.5 51.5) (end 115 51.5) (width 0.2) (layer "F.Cu") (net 33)))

